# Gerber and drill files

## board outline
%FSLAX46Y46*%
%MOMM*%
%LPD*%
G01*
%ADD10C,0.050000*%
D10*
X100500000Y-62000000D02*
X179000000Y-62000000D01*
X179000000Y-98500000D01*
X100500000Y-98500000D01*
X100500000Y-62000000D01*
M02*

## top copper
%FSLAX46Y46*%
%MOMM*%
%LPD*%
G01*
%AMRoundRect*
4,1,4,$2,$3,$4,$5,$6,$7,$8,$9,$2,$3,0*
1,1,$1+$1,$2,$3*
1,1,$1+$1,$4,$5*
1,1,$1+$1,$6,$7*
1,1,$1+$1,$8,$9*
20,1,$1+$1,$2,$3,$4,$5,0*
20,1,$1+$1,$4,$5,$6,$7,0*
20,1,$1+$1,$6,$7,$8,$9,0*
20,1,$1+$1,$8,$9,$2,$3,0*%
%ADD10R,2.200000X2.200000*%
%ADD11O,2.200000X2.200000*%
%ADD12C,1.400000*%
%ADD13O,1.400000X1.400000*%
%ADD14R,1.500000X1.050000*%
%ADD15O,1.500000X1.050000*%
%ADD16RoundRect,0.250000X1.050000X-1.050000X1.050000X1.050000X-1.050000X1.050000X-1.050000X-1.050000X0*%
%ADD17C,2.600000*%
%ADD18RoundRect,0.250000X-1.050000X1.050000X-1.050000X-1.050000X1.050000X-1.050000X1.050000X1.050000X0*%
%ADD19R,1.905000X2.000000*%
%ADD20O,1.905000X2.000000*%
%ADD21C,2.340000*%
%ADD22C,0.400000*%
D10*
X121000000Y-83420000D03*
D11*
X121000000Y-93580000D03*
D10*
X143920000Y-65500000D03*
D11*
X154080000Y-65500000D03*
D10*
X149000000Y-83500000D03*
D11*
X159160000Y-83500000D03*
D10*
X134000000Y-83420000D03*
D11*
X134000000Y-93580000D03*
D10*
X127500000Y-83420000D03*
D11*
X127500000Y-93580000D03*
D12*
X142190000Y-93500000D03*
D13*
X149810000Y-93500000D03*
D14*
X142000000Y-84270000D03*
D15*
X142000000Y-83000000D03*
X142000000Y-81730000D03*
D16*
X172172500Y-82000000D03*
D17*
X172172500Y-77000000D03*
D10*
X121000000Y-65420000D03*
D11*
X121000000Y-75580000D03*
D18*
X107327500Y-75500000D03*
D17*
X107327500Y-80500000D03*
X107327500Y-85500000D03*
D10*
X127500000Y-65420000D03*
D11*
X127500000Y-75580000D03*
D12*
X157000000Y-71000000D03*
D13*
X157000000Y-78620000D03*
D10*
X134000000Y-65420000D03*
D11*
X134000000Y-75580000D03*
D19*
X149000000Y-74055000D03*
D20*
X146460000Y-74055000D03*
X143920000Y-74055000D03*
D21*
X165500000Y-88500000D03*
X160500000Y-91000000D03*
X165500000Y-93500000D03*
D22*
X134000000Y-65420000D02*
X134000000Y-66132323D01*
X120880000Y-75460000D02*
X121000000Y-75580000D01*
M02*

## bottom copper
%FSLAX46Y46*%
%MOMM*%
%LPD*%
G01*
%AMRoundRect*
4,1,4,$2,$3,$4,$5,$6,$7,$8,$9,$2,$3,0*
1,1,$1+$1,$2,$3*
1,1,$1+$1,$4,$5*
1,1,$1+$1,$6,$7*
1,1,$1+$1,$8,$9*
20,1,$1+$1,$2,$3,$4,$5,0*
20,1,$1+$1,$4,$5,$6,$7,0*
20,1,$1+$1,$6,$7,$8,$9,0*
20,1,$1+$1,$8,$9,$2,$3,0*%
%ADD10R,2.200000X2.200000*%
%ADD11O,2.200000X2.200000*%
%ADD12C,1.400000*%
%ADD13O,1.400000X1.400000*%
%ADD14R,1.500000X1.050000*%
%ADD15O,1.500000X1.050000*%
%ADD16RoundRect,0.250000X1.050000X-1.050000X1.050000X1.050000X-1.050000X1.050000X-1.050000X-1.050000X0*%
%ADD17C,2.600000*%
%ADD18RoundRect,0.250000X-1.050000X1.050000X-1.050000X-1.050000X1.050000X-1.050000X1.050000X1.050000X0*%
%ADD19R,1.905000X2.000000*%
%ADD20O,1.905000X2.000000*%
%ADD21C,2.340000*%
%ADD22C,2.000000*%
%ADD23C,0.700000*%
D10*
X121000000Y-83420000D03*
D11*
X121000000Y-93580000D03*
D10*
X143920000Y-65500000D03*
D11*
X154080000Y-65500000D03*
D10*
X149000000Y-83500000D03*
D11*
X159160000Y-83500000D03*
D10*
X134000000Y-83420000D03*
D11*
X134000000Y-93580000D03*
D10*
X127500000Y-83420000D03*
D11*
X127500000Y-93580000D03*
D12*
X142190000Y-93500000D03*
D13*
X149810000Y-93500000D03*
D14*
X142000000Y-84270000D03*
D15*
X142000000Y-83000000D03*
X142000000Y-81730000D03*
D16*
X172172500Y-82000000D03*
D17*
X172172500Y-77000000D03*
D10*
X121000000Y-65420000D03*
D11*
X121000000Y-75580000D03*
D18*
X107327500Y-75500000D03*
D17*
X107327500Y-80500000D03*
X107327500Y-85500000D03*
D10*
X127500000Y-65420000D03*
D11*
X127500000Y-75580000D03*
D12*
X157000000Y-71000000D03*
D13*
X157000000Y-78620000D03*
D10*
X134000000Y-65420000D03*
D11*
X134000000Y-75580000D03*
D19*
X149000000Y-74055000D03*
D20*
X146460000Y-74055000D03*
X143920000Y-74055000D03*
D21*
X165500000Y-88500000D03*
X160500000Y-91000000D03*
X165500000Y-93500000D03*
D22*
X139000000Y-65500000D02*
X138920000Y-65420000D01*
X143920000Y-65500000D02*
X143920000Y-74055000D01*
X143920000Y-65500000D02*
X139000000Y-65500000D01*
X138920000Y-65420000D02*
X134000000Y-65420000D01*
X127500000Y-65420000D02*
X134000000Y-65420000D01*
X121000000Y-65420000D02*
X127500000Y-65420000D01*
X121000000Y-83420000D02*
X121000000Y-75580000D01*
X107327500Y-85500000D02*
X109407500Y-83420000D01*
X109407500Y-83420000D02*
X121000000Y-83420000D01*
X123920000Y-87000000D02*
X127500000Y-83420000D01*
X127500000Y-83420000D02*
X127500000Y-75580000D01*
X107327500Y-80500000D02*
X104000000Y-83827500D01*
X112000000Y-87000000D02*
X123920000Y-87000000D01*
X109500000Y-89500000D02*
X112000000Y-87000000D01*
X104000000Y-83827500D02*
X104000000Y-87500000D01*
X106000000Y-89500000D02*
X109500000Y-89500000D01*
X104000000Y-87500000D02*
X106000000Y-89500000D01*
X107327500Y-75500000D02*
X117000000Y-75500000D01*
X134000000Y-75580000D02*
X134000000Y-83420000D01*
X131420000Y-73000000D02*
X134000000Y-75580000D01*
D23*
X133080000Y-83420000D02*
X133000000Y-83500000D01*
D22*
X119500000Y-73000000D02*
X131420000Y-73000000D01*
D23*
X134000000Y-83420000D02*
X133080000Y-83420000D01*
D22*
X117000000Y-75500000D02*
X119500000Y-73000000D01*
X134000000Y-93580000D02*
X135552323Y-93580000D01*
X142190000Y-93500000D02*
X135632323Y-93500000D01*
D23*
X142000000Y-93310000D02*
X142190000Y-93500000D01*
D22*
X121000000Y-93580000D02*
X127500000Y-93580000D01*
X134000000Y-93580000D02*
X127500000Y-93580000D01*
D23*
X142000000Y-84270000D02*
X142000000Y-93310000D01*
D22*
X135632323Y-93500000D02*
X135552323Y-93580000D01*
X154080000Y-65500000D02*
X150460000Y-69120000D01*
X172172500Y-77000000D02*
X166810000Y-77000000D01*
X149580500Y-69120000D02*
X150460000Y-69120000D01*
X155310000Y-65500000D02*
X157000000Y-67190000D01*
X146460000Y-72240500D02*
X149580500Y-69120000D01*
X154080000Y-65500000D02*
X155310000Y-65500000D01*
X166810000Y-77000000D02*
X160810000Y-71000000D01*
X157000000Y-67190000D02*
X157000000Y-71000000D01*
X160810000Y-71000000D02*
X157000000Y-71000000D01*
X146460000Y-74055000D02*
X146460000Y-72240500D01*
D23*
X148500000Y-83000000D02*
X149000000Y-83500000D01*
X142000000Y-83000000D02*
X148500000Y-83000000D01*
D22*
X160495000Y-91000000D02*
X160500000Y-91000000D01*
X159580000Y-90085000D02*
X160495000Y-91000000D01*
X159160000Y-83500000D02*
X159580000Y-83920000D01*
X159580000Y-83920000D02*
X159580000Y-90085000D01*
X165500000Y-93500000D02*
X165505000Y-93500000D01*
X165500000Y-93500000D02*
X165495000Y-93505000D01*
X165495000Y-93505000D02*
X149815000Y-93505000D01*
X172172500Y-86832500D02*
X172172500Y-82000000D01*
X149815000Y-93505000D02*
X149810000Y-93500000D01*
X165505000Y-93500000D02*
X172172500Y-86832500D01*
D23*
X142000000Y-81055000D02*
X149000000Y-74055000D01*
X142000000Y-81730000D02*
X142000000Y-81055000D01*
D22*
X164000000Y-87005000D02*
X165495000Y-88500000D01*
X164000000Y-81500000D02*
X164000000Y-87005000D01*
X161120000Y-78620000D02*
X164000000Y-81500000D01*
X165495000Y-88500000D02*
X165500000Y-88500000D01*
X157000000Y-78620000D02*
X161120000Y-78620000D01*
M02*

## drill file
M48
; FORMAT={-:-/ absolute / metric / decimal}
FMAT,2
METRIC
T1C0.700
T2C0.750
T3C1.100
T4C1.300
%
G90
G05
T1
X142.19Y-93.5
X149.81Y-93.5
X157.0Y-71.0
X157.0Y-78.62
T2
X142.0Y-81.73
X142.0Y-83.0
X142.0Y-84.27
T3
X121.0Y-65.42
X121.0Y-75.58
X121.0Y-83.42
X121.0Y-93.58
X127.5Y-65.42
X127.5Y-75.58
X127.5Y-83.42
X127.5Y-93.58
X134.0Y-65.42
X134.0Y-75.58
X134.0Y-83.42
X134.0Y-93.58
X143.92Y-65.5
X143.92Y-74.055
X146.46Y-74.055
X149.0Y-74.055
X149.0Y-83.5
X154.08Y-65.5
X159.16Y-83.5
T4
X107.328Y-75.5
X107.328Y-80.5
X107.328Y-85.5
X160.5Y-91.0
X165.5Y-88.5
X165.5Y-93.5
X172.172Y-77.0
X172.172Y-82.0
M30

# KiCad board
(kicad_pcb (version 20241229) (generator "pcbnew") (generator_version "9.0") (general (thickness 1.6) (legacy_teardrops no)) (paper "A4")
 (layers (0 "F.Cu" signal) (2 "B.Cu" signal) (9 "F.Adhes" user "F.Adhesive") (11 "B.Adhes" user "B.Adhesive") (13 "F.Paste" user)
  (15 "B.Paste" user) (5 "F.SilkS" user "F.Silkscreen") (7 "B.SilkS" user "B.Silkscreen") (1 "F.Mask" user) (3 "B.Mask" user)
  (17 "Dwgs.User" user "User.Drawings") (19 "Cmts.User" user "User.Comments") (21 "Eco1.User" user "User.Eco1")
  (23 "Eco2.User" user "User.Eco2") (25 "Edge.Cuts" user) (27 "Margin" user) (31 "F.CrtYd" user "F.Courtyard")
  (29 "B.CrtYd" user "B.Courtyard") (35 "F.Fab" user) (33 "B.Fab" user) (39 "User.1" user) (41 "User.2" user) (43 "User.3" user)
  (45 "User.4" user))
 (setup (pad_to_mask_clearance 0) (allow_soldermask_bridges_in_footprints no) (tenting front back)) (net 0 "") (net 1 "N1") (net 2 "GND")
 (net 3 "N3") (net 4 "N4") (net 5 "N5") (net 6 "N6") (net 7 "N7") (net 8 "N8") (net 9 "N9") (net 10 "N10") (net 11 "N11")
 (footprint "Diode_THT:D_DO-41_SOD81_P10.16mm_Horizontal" (layer "F.Cu") (at 121 83.42 -90)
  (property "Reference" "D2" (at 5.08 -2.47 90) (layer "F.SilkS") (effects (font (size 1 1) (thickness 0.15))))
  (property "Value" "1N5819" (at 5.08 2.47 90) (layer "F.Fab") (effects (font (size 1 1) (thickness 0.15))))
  (pad "1" thru_hole rect (at 0 0 270) (size 2.2 2.2) (drill 1.1) (layers "*.Cu" "*.Mask") (remove_unused_layers no) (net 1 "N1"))
  (pad "2" thru_hole oval (at 10.16 0 270) (size 2.2 2.2) (drill 1.1) (layers "*.Cu" "*.Mask") (remove_unused_layers no) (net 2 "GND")))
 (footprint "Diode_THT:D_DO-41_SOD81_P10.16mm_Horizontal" (layer "F.Cu") (at 143.92 65.5)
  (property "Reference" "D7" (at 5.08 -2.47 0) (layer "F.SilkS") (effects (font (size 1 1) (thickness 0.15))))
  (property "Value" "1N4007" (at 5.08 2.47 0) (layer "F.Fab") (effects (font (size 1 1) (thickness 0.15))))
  (pad "1" thru_hole rect (at 0 0) (size 2.2 2.2) (drill 1.1) (layers "*.Cu" "*.Mask") (remove_unused_layers no) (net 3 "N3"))
  (pad "2" thru_hole oval (at 10.16 0) (size 2.2 2.2) (drill 1.1) (layers "*.Cu" "*.Mask") (remove_unused_layers no) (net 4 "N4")))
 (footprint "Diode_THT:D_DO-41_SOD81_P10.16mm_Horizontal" (layer "F.Cu") (at 149 83.5)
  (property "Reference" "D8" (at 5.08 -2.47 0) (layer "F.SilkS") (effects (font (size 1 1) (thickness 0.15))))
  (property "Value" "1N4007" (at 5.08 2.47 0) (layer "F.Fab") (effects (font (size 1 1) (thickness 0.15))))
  (pad "1" thru_hole rect (at 0 0) (size 2.2 2.2) (drill 1.1) (layers "*.Cu" "*.Mask") (remove_unused_layers no) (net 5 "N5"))
  (pad "2" thru_hole oval (at 10.16 0) (size 2.2 2.2) (drill 1.1) (layers "*.Cu" "*.Mask") (remove_unused_layers no) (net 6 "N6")))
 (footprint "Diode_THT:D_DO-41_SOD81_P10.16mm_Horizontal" (layer "F.Cu") (at 134 83.42 -90)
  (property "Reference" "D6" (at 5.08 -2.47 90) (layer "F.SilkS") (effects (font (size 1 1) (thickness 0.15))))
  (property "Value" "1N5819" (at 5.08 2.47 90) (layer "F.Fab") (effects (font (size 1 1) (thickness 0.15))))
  (pad "1" thru_hole rect (at 0 0 270) (size 2.2 2.2) (drill 1.1) (layers "*.Cu" "*.Mask") (remove_unused_layers no) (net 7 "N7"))
  (pad "2" thru_hole oval (at 10.16 0 270) (size 2.2 2.2) (drill 1.1) (layers "*.Cu" "*.Mask") (remove_unused_layers no) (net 2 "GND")))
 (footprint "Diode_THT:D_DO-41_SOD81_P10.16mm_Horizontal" (layer "F.Cu") (at 127.5 83.42 -90)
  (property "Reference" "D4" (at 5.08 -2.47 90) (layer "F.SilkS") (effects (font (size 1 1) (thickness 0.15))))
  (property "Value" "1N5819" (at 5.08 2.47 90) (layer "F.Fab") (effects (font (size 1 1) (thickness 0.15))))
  (pad "1" thru_hole rect (at 0 0 270) (size 2.2 2.2) (drill 1.1) (layers "*.Cu" "*.Mask") (remove_unused_layers no) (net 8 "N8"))
  (pad "2" thru_hole oval (at 10.16 0 270) (size 2.2 2.2) (drill 1.1) (layers "*.Cu" "*.Mask") (remove_unused_layers no) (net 2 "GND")))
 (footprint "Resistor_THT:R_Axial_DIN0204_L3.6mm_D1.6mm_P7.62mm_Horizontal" (layer "F.Cu") (at 142.19 93.5)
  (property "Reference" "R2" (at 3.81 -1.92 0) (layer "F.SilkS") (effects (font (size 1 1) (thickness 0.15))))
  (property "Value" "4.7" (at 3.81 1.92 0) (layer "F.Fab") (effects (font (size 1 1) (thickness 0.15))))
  (pad "1" thru_hole circle (at 0 0) (size 1.4 1.4) (drill 0.7) (layers "*.Cu" "*.Mask") (remove_unused_layers no) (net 2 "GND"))
  (pad "2" thru_hole oval (at 7.62 0) (size 1.4 1.4) (drill 0.7) (layers "*.Cu" "*.Mask") (remove_unused_layers no) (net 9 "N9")))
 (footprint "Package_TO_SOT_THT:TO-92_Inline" (layer "F.Cu") (at 142 84.27 90)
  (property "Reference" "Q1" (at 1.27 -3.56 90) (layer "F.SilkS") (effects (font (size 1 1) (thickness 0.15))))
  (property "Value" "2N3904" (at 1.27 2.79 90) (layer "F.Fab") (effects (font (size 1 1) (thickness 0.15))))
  (pad "1" thru_hole rect (at 0 0 90) (size 1.05 1.5) (drill 0.75) (layers "*.Cu" "*.Mask") (remove_unused_layers no) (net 2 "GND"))
  (pad "2" thru_hole oval (at 1.27 0 90) (size 1.05 1.5) (drill 0.75) (layers "*.Cu" "*.Mask") (remove_unused_layers no) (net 5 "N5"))
  (pad "3" thru_hole oval (at 2.54 0 90) (size 1.05 1.5) (drill 0.75) (layers "*.Cu" "*.Mask") (remove_unused_layers no) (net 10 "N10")))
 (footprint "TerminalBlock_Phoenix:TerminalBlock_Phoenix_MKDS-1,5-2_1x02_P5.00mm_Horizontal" (layer "F.Cu") (at 172.1725 82 90)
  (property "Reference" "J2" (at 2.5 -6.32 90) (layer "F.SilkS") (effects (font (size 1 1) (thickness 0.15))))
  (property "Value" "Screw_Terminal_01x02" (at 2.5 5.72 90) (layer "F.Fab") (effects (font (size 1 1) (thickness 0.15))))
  (pad "1" thru_hole roundrect (at 0 0 90) (size 2.6 2.6) (drill 1.3) (layers "*.Cu" "*.Mask") (remove_unused_layers no)
   (roundrect_rratio 0.096154) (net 9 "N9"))
  (pad "2" thru_hole circle (at 5 0 90) (size 2.6 2.6) (drill 1.3) (layers "*.Cu" "*.Mask") (remove_unused_layers no) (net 4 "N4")))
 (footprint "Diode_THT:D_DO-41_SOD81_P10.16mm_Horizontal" (layer "F.Cu") (at 121 65.42 -90)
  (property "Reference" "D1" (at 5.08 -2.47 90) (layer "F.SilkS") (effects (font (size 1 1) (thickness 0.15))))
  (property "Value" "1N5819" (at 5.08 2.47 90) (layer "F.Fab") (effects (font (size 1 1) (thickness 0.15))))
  (pad "1" thru_hole rect (at 0 0 270) (size 2.2 2.2) (drill 1.1) (layers "*.Cu" "*.Mask") (remove_unused_layers no) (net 3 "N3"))
  (pad "2" thru_hole oval (at 10.16 0 270) (size 2.2 2.2) (drill 1.1) (layers "*.Cu" "*.Mask") (remove_unused_layers no) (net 1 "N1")))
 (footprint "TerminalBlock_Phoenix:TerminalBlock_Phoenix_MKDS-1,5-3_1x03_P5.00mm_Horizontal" (layer "F.Cu") (at 107.3275 75.5 -90)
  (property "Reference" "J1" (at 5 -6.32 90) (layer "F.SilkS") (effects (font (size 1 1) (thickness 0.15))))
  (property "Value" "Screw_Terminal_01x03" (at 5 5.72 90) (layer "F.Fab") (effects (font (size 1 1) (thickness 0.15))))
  (pad "1" thru_hole roundrect (at 0 0 270) (size 2.6 2.6) (drill 1.3) (layers "*.Cu" "*.Mask") (remove_unused_layers no)
   (roundrect_rratio 0.096154) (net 7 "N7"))
  (pad "2" thru_hole circle (at 5 0 270) (size 2.6 2.6) (drill 1.3) (layers "*.Cu" "*.Mask") (remove_unused_layers no) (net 8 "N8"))
  (pad "3" thru_hole circle (at 10 0 270) (size 2.6 2.6) (drill 1.3) (layers "*.Cu" "*.Mask") (remove_unused_layers no) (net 1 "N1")))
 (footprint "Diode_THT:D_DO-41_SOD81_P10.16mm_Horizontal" (layer "F.Cu") (at 127.5 65.42 -90)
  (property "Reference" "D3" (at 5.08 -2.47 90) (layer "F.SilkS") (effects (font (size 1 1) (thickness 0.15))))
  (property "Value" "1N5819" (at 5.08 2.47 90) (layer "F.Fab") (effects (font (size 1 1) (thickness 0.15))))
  (pad "1" thru_hole rect (at 0 0 270) (size 2.2 2.2) (drill 1.1) (layers "*.Cu" "*.Mask") (remove_unused_layers no) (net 3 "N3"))
  (pad "2" thru_hole oval (at 10.16 0 270) (size 2.2 2.2) (drill 1.1) (layers "*.Cu" "*.Mask") (remove_unused_layers no) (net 8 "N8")))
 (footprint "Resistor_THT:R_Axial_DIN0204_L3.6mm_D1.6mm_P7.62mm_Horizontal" (layer "F.Cu") (at 157 71 -90)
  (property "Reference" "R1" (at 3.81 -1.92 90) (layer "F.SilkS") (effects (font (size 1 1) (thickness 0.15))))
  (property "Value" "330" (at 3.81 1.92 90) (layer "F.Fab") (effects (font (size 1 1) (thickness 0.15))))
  (pad "1" thru_hole circle (at 0 0 270) (size 1.4 1.4) (drill 0.7) (layers "*.Cu" "*.Mask") (remove_unused_layers no) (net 4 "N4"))
  (pad "2" thru_hole oval (at 7.62 0 270) (size 1.4 1.4) (drill 0.7) (layers "*.Cu" "*.Mask") (remove_unused_layers no) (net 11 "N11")))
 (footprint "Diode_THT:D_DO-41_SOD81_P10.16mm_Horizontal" (layer "F.Cu") (at 134 65.42 -90)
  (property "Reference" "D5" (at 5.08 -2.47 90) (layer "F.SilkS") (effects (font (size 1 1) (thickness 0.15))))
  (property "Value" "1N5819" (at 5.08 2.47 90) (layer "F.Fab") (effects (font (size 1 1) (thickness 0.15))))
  (pad "1" thru_hole rect (at 0 0 270) (size 2.2 2.2) (drill 1.1) (layers "*.Cu" "*.Mask") (remove_unused_layers no) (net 3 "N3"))
  (pad "2" thru_hole oval (at 10.16 0 270) (size 2.2 2.2) (drill 1.1) (layers "*.Cu" "*.Mask") (remove_unused_layers no) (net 7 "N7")))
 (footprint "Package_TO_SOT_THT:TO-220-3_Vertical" (layer "F.Cu") (at 149 74.055 180)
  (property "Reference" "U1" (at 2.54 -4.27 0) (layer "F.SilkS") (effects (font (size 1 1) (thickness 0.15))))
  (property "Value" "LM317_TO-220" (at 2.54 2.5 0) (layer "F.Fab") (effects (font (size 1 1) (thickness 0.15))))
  (pad "1" thru_hole rect (at 0 0 180) (size 1.905 2) (drill 1.1) (layers "*.Cu" "*.Mask") (remove_unused_layers no) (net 10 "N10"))
  (pad "2" thru_hole oval (at 2.54 0 180) (size 1.905 2) (drill 1.1) (layers "*.Cu" "*.Mask") (remove_unused_layers no) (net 4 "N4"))
  (pad "3" thru_hole oval (at 5.08 0 180) (size 1.905 2) (drill 1.1) (layers "*.Cu" "*.Mask") (remove_unused_layers no) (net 3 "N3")))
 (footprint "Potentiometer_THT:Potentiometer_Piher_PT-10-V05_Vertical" (layer "F.Cu") (at 165.5 88.5 180)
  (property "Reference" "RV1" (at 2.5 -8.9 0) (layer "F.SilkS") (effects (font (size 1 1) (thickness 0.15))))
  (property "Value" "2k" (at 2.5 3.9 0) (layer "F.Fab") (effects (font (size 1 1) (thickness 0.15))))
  (pad "1" thru_hole circle (at 0 0 180) (size 2.34 2.34) (drill 1.3) (layers "*.Cu" "*.Mask") (remove_unused_layers no) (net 11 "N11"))
  (pad "2" thru_hole circle (at 5 -2.5 180) (size 2.34 2.34) (drill 1.3) (layers "*.Cu" "*.Mask") (remove_unused_layers no) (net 6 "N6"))
  (pad "3" thru_hole circle (at 0 -5 180) (size 2.34 2.34) (drill 1.3) (layers "*.Cu" "*.Mask") (remove_unused_layers no) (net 9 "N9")))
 (gr_rect (start 100.5 62) (end 179 98.5) (stroke (width 0.05) (type default)) (fill no) (layer "Edge.Cuts"))
 (segment (start 134 65.42) (end 134 66.132323) (width 0.4) (layer "F.Cu") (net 3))
 (segment (start 139 65.5) (end 138.92 65.42) (width 2) (layer "B.Cu") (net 3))
 (segment (start 143.92 65.5) (end 143.92 74.055) (width 2) (layer "B.Cu") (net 3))
 (segment (start 143.92 65.5) (end 139 65.5) (width 2) (layer "B.Cu") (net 3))
 (segment (start 138.92 65.42) (end 134 65.42) (width 2) (layer "B.Cu") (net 3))
 (segment (start 127.5 65.42) (end 134 65.42) (width 2) (layer "B.Cu") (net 3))
 (segment (start 121 65.42) (end 127.5 65.42) (width 2) (layer "B.Cu") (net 3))
 (segment (start 120.88 75.46) (end 121 75.58) (width 0.4) (layer "F.Cu") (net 1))
 (segment (start 121 83.42) (end 121 75.58) (width 2) (layer "B.Cu") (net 1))
 (segment (start 107.3275 85.5) (end 109.4075 83.42) (width 2) (layer "B.Cu") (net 1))
 (segment (start 109.4075 83.42) (end 121 83.42) (width 2) (layer "B.Cu") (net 1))
 (segment (start 123.92 87) (end 127.5 83.42) (width 2) (layer "B.Cu") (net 8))
 (segment (start 127.5 83.42) (end 127.5 75.58) (width 2) (layer "B.Cu") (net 8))
 (segment (start 107.3275 80.5) (end 104 83.8275) (width 2) (layer "B.Cu") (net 8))
 (segment (start 112 87) (end 123.92 87) (width 2) (layer "B.Cu") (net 8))
 (segment (start 109.5 89.5) (end 112 87) (width 2) (layer "B.Cu") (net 8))
 (segment (start 104 83.8275) (end 104 87.5) (width 2) (layer "B.Cu") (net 8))
 (segment (start 106 89.5) (end 109.5 89.5) (width 2) (layer "B.Cu") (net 8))
 (segment (start 104 87.5) (end 106 89.5) (width 2) (layer "B.Cu") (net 8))
 (segment (start 107.3275 75.5) (end 117 75.5) (width 2) (layer "B.Cu") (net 7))
 (segment (start 134 75.58) (end 134 83.42) (width 2) (layer "B.Cu") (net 7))
 (segment (start 131.42 73) (end 134 75.58) (width 2) (layer "B.Cu") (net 7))
 (segment (start 133.08 83.42) (end 133 83.5) (width 0.7) (layer "B.Cu") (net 7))
 (segment (start 119.5 73) (end 131.42 73) (width 2) (layer "B.Cu") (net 7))
 (segment (start 134 83.42) (end 133.08 83.42) (width 0.7) (layer "B.Cu") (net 7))
 (segment (start 117 75.5) (end 119.5 73) (width 2) (layer "B.Cu") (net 7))
 (segment (start 134 93.58) (end 135.552323 93.58) (width 2) (layer "B.Cu") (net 2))
 (segment (start 142.19 93.5) (end 135.632323 93.5) (width 2) (layer "B.Cu") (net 2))
 (segment (start 142 93.31) (end 142.19 93.5) (width 0.7) (layer "B.Cu") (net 2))
 (segment (start 121 93.58) (end 127.5 93.58) (width 2) (layer "B.Cu") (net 2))
 (segment (start 134 93.58) (end 127.5 93.58) (width 2) (layer "B.Cu") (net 2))
 (segment (start 142 84.27) (end 142 93.31) (width 0.7) (layer "B.Cu") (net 2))
 (segment (start 135.632323 93.5) (end 135.552323 93.58) (width 2) (layer "B.Cu") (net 2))
 (segment (start 154.08 65.5) (end 150.46 69.12) (width 2) (layer "B.Cu") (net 4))
 (segment (start 172.1725 77) (end 166.81 77) (width 2) (layer "B.Cu") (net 4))
 (segment (start 149.5805 69.12) (end 150.46 69.12) (width 2) (layer "B.Cu") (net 4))
 (segment (start 155.31 65.5) (end 157 67.19) (width 2) (layer "B.Cu") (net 4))
 (segment (start 146.46 72.2405) (end 149.5805 69.12) (width 2) (layer "B.Cu") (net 4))
 (segment (start 154.08 65.5) (end 155.31 65.5) (width 2) (layer "B.Cu") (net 4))
 (segment (start 166.81 77) (end 160.81 71) (width 2) (layer "B.Cu") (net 4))
 (segment (start 157 67.19) (end 157 71) (width 2) (layer "B.Cu") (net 4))
 (segment (start 160.81 71) (end 157 71) (width 2) (layer "B.Cu") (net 4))
 (segment (start 146.46 74.055) (end 146.46 72.2405) (width 2) (layer "B.Cu") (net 4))
 (segment (start 148.5 83) (end 149 83.5) (width 0.7) (layer "B.Cu") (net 5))
 (segment (start 142 83) (end 148.5 83) (width 0.7) (layer "B.Cu") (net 5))
 (segment (start 160.495 91) (end 160.5 91) (width 2) (layer "B.Cu") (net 6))
 (segment (start 159.58 90.085) (end 160.495 91) (width 2) (layer "B.Cu") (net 6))
 (segment (start 159.16 83.5) (end 159.58 83.92) (width 2) (layer "B.Cu") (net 6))
 (segment (start 159.58 83.92) (end 159.58 90.085) (width 2) (layer "B.Cu") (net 6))
 (segment (start 165.5 93.5) (end 165.505 93.5) (width 2) (layer "B.Cu") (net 9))
 (segment (start 165.5 93.5) (end 165.495 93.505) (width 2) (layer "B.Cu") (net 9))
 (segment (start 165.495 93.505) (end 149.815 93.505) (width 2) (layer "B.Cu") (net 9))
 (segment (start 172.1725 86.8325) (end 172.1725 82) (width 2) (layer "B.Cu") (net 9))
 (segment (start 149.815 93.505) (end 149.81 93.5) (width 2) (layer "B.Cu") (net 9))
 (segment (start 165.505 93.5) (end 172.1725 86.8325) (width 2) (layer "B.Cu") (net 9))
 (segment (start 142 81.055) (end 149 74.055) (width 0.7) (layer "B.Cu") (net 10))
 (segment (start 142 81.73) (end 142 81.055) (width 0.7) (layer "B.Cu") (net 10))
 (segment (start 164 87.005) (end 165.495 88.5) (width 2) (layer "B.Cu") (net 11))
 (segment (start 164 81.5) (end 164 87.005) (width 2) (layer "B.Cu") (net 11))
 (segment (start 161.12 78.62) (end 164 81.5) (width 2) (layer "B.Cu") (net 11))
 (segment (start 165.495 88.5) (end 165.5 88.5) (width 2) (layer "B.Cu") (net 11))
 (segment (start 157 78.62) (end 161.12 78.62) (width 2) (layer "B.Cu") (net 11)))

